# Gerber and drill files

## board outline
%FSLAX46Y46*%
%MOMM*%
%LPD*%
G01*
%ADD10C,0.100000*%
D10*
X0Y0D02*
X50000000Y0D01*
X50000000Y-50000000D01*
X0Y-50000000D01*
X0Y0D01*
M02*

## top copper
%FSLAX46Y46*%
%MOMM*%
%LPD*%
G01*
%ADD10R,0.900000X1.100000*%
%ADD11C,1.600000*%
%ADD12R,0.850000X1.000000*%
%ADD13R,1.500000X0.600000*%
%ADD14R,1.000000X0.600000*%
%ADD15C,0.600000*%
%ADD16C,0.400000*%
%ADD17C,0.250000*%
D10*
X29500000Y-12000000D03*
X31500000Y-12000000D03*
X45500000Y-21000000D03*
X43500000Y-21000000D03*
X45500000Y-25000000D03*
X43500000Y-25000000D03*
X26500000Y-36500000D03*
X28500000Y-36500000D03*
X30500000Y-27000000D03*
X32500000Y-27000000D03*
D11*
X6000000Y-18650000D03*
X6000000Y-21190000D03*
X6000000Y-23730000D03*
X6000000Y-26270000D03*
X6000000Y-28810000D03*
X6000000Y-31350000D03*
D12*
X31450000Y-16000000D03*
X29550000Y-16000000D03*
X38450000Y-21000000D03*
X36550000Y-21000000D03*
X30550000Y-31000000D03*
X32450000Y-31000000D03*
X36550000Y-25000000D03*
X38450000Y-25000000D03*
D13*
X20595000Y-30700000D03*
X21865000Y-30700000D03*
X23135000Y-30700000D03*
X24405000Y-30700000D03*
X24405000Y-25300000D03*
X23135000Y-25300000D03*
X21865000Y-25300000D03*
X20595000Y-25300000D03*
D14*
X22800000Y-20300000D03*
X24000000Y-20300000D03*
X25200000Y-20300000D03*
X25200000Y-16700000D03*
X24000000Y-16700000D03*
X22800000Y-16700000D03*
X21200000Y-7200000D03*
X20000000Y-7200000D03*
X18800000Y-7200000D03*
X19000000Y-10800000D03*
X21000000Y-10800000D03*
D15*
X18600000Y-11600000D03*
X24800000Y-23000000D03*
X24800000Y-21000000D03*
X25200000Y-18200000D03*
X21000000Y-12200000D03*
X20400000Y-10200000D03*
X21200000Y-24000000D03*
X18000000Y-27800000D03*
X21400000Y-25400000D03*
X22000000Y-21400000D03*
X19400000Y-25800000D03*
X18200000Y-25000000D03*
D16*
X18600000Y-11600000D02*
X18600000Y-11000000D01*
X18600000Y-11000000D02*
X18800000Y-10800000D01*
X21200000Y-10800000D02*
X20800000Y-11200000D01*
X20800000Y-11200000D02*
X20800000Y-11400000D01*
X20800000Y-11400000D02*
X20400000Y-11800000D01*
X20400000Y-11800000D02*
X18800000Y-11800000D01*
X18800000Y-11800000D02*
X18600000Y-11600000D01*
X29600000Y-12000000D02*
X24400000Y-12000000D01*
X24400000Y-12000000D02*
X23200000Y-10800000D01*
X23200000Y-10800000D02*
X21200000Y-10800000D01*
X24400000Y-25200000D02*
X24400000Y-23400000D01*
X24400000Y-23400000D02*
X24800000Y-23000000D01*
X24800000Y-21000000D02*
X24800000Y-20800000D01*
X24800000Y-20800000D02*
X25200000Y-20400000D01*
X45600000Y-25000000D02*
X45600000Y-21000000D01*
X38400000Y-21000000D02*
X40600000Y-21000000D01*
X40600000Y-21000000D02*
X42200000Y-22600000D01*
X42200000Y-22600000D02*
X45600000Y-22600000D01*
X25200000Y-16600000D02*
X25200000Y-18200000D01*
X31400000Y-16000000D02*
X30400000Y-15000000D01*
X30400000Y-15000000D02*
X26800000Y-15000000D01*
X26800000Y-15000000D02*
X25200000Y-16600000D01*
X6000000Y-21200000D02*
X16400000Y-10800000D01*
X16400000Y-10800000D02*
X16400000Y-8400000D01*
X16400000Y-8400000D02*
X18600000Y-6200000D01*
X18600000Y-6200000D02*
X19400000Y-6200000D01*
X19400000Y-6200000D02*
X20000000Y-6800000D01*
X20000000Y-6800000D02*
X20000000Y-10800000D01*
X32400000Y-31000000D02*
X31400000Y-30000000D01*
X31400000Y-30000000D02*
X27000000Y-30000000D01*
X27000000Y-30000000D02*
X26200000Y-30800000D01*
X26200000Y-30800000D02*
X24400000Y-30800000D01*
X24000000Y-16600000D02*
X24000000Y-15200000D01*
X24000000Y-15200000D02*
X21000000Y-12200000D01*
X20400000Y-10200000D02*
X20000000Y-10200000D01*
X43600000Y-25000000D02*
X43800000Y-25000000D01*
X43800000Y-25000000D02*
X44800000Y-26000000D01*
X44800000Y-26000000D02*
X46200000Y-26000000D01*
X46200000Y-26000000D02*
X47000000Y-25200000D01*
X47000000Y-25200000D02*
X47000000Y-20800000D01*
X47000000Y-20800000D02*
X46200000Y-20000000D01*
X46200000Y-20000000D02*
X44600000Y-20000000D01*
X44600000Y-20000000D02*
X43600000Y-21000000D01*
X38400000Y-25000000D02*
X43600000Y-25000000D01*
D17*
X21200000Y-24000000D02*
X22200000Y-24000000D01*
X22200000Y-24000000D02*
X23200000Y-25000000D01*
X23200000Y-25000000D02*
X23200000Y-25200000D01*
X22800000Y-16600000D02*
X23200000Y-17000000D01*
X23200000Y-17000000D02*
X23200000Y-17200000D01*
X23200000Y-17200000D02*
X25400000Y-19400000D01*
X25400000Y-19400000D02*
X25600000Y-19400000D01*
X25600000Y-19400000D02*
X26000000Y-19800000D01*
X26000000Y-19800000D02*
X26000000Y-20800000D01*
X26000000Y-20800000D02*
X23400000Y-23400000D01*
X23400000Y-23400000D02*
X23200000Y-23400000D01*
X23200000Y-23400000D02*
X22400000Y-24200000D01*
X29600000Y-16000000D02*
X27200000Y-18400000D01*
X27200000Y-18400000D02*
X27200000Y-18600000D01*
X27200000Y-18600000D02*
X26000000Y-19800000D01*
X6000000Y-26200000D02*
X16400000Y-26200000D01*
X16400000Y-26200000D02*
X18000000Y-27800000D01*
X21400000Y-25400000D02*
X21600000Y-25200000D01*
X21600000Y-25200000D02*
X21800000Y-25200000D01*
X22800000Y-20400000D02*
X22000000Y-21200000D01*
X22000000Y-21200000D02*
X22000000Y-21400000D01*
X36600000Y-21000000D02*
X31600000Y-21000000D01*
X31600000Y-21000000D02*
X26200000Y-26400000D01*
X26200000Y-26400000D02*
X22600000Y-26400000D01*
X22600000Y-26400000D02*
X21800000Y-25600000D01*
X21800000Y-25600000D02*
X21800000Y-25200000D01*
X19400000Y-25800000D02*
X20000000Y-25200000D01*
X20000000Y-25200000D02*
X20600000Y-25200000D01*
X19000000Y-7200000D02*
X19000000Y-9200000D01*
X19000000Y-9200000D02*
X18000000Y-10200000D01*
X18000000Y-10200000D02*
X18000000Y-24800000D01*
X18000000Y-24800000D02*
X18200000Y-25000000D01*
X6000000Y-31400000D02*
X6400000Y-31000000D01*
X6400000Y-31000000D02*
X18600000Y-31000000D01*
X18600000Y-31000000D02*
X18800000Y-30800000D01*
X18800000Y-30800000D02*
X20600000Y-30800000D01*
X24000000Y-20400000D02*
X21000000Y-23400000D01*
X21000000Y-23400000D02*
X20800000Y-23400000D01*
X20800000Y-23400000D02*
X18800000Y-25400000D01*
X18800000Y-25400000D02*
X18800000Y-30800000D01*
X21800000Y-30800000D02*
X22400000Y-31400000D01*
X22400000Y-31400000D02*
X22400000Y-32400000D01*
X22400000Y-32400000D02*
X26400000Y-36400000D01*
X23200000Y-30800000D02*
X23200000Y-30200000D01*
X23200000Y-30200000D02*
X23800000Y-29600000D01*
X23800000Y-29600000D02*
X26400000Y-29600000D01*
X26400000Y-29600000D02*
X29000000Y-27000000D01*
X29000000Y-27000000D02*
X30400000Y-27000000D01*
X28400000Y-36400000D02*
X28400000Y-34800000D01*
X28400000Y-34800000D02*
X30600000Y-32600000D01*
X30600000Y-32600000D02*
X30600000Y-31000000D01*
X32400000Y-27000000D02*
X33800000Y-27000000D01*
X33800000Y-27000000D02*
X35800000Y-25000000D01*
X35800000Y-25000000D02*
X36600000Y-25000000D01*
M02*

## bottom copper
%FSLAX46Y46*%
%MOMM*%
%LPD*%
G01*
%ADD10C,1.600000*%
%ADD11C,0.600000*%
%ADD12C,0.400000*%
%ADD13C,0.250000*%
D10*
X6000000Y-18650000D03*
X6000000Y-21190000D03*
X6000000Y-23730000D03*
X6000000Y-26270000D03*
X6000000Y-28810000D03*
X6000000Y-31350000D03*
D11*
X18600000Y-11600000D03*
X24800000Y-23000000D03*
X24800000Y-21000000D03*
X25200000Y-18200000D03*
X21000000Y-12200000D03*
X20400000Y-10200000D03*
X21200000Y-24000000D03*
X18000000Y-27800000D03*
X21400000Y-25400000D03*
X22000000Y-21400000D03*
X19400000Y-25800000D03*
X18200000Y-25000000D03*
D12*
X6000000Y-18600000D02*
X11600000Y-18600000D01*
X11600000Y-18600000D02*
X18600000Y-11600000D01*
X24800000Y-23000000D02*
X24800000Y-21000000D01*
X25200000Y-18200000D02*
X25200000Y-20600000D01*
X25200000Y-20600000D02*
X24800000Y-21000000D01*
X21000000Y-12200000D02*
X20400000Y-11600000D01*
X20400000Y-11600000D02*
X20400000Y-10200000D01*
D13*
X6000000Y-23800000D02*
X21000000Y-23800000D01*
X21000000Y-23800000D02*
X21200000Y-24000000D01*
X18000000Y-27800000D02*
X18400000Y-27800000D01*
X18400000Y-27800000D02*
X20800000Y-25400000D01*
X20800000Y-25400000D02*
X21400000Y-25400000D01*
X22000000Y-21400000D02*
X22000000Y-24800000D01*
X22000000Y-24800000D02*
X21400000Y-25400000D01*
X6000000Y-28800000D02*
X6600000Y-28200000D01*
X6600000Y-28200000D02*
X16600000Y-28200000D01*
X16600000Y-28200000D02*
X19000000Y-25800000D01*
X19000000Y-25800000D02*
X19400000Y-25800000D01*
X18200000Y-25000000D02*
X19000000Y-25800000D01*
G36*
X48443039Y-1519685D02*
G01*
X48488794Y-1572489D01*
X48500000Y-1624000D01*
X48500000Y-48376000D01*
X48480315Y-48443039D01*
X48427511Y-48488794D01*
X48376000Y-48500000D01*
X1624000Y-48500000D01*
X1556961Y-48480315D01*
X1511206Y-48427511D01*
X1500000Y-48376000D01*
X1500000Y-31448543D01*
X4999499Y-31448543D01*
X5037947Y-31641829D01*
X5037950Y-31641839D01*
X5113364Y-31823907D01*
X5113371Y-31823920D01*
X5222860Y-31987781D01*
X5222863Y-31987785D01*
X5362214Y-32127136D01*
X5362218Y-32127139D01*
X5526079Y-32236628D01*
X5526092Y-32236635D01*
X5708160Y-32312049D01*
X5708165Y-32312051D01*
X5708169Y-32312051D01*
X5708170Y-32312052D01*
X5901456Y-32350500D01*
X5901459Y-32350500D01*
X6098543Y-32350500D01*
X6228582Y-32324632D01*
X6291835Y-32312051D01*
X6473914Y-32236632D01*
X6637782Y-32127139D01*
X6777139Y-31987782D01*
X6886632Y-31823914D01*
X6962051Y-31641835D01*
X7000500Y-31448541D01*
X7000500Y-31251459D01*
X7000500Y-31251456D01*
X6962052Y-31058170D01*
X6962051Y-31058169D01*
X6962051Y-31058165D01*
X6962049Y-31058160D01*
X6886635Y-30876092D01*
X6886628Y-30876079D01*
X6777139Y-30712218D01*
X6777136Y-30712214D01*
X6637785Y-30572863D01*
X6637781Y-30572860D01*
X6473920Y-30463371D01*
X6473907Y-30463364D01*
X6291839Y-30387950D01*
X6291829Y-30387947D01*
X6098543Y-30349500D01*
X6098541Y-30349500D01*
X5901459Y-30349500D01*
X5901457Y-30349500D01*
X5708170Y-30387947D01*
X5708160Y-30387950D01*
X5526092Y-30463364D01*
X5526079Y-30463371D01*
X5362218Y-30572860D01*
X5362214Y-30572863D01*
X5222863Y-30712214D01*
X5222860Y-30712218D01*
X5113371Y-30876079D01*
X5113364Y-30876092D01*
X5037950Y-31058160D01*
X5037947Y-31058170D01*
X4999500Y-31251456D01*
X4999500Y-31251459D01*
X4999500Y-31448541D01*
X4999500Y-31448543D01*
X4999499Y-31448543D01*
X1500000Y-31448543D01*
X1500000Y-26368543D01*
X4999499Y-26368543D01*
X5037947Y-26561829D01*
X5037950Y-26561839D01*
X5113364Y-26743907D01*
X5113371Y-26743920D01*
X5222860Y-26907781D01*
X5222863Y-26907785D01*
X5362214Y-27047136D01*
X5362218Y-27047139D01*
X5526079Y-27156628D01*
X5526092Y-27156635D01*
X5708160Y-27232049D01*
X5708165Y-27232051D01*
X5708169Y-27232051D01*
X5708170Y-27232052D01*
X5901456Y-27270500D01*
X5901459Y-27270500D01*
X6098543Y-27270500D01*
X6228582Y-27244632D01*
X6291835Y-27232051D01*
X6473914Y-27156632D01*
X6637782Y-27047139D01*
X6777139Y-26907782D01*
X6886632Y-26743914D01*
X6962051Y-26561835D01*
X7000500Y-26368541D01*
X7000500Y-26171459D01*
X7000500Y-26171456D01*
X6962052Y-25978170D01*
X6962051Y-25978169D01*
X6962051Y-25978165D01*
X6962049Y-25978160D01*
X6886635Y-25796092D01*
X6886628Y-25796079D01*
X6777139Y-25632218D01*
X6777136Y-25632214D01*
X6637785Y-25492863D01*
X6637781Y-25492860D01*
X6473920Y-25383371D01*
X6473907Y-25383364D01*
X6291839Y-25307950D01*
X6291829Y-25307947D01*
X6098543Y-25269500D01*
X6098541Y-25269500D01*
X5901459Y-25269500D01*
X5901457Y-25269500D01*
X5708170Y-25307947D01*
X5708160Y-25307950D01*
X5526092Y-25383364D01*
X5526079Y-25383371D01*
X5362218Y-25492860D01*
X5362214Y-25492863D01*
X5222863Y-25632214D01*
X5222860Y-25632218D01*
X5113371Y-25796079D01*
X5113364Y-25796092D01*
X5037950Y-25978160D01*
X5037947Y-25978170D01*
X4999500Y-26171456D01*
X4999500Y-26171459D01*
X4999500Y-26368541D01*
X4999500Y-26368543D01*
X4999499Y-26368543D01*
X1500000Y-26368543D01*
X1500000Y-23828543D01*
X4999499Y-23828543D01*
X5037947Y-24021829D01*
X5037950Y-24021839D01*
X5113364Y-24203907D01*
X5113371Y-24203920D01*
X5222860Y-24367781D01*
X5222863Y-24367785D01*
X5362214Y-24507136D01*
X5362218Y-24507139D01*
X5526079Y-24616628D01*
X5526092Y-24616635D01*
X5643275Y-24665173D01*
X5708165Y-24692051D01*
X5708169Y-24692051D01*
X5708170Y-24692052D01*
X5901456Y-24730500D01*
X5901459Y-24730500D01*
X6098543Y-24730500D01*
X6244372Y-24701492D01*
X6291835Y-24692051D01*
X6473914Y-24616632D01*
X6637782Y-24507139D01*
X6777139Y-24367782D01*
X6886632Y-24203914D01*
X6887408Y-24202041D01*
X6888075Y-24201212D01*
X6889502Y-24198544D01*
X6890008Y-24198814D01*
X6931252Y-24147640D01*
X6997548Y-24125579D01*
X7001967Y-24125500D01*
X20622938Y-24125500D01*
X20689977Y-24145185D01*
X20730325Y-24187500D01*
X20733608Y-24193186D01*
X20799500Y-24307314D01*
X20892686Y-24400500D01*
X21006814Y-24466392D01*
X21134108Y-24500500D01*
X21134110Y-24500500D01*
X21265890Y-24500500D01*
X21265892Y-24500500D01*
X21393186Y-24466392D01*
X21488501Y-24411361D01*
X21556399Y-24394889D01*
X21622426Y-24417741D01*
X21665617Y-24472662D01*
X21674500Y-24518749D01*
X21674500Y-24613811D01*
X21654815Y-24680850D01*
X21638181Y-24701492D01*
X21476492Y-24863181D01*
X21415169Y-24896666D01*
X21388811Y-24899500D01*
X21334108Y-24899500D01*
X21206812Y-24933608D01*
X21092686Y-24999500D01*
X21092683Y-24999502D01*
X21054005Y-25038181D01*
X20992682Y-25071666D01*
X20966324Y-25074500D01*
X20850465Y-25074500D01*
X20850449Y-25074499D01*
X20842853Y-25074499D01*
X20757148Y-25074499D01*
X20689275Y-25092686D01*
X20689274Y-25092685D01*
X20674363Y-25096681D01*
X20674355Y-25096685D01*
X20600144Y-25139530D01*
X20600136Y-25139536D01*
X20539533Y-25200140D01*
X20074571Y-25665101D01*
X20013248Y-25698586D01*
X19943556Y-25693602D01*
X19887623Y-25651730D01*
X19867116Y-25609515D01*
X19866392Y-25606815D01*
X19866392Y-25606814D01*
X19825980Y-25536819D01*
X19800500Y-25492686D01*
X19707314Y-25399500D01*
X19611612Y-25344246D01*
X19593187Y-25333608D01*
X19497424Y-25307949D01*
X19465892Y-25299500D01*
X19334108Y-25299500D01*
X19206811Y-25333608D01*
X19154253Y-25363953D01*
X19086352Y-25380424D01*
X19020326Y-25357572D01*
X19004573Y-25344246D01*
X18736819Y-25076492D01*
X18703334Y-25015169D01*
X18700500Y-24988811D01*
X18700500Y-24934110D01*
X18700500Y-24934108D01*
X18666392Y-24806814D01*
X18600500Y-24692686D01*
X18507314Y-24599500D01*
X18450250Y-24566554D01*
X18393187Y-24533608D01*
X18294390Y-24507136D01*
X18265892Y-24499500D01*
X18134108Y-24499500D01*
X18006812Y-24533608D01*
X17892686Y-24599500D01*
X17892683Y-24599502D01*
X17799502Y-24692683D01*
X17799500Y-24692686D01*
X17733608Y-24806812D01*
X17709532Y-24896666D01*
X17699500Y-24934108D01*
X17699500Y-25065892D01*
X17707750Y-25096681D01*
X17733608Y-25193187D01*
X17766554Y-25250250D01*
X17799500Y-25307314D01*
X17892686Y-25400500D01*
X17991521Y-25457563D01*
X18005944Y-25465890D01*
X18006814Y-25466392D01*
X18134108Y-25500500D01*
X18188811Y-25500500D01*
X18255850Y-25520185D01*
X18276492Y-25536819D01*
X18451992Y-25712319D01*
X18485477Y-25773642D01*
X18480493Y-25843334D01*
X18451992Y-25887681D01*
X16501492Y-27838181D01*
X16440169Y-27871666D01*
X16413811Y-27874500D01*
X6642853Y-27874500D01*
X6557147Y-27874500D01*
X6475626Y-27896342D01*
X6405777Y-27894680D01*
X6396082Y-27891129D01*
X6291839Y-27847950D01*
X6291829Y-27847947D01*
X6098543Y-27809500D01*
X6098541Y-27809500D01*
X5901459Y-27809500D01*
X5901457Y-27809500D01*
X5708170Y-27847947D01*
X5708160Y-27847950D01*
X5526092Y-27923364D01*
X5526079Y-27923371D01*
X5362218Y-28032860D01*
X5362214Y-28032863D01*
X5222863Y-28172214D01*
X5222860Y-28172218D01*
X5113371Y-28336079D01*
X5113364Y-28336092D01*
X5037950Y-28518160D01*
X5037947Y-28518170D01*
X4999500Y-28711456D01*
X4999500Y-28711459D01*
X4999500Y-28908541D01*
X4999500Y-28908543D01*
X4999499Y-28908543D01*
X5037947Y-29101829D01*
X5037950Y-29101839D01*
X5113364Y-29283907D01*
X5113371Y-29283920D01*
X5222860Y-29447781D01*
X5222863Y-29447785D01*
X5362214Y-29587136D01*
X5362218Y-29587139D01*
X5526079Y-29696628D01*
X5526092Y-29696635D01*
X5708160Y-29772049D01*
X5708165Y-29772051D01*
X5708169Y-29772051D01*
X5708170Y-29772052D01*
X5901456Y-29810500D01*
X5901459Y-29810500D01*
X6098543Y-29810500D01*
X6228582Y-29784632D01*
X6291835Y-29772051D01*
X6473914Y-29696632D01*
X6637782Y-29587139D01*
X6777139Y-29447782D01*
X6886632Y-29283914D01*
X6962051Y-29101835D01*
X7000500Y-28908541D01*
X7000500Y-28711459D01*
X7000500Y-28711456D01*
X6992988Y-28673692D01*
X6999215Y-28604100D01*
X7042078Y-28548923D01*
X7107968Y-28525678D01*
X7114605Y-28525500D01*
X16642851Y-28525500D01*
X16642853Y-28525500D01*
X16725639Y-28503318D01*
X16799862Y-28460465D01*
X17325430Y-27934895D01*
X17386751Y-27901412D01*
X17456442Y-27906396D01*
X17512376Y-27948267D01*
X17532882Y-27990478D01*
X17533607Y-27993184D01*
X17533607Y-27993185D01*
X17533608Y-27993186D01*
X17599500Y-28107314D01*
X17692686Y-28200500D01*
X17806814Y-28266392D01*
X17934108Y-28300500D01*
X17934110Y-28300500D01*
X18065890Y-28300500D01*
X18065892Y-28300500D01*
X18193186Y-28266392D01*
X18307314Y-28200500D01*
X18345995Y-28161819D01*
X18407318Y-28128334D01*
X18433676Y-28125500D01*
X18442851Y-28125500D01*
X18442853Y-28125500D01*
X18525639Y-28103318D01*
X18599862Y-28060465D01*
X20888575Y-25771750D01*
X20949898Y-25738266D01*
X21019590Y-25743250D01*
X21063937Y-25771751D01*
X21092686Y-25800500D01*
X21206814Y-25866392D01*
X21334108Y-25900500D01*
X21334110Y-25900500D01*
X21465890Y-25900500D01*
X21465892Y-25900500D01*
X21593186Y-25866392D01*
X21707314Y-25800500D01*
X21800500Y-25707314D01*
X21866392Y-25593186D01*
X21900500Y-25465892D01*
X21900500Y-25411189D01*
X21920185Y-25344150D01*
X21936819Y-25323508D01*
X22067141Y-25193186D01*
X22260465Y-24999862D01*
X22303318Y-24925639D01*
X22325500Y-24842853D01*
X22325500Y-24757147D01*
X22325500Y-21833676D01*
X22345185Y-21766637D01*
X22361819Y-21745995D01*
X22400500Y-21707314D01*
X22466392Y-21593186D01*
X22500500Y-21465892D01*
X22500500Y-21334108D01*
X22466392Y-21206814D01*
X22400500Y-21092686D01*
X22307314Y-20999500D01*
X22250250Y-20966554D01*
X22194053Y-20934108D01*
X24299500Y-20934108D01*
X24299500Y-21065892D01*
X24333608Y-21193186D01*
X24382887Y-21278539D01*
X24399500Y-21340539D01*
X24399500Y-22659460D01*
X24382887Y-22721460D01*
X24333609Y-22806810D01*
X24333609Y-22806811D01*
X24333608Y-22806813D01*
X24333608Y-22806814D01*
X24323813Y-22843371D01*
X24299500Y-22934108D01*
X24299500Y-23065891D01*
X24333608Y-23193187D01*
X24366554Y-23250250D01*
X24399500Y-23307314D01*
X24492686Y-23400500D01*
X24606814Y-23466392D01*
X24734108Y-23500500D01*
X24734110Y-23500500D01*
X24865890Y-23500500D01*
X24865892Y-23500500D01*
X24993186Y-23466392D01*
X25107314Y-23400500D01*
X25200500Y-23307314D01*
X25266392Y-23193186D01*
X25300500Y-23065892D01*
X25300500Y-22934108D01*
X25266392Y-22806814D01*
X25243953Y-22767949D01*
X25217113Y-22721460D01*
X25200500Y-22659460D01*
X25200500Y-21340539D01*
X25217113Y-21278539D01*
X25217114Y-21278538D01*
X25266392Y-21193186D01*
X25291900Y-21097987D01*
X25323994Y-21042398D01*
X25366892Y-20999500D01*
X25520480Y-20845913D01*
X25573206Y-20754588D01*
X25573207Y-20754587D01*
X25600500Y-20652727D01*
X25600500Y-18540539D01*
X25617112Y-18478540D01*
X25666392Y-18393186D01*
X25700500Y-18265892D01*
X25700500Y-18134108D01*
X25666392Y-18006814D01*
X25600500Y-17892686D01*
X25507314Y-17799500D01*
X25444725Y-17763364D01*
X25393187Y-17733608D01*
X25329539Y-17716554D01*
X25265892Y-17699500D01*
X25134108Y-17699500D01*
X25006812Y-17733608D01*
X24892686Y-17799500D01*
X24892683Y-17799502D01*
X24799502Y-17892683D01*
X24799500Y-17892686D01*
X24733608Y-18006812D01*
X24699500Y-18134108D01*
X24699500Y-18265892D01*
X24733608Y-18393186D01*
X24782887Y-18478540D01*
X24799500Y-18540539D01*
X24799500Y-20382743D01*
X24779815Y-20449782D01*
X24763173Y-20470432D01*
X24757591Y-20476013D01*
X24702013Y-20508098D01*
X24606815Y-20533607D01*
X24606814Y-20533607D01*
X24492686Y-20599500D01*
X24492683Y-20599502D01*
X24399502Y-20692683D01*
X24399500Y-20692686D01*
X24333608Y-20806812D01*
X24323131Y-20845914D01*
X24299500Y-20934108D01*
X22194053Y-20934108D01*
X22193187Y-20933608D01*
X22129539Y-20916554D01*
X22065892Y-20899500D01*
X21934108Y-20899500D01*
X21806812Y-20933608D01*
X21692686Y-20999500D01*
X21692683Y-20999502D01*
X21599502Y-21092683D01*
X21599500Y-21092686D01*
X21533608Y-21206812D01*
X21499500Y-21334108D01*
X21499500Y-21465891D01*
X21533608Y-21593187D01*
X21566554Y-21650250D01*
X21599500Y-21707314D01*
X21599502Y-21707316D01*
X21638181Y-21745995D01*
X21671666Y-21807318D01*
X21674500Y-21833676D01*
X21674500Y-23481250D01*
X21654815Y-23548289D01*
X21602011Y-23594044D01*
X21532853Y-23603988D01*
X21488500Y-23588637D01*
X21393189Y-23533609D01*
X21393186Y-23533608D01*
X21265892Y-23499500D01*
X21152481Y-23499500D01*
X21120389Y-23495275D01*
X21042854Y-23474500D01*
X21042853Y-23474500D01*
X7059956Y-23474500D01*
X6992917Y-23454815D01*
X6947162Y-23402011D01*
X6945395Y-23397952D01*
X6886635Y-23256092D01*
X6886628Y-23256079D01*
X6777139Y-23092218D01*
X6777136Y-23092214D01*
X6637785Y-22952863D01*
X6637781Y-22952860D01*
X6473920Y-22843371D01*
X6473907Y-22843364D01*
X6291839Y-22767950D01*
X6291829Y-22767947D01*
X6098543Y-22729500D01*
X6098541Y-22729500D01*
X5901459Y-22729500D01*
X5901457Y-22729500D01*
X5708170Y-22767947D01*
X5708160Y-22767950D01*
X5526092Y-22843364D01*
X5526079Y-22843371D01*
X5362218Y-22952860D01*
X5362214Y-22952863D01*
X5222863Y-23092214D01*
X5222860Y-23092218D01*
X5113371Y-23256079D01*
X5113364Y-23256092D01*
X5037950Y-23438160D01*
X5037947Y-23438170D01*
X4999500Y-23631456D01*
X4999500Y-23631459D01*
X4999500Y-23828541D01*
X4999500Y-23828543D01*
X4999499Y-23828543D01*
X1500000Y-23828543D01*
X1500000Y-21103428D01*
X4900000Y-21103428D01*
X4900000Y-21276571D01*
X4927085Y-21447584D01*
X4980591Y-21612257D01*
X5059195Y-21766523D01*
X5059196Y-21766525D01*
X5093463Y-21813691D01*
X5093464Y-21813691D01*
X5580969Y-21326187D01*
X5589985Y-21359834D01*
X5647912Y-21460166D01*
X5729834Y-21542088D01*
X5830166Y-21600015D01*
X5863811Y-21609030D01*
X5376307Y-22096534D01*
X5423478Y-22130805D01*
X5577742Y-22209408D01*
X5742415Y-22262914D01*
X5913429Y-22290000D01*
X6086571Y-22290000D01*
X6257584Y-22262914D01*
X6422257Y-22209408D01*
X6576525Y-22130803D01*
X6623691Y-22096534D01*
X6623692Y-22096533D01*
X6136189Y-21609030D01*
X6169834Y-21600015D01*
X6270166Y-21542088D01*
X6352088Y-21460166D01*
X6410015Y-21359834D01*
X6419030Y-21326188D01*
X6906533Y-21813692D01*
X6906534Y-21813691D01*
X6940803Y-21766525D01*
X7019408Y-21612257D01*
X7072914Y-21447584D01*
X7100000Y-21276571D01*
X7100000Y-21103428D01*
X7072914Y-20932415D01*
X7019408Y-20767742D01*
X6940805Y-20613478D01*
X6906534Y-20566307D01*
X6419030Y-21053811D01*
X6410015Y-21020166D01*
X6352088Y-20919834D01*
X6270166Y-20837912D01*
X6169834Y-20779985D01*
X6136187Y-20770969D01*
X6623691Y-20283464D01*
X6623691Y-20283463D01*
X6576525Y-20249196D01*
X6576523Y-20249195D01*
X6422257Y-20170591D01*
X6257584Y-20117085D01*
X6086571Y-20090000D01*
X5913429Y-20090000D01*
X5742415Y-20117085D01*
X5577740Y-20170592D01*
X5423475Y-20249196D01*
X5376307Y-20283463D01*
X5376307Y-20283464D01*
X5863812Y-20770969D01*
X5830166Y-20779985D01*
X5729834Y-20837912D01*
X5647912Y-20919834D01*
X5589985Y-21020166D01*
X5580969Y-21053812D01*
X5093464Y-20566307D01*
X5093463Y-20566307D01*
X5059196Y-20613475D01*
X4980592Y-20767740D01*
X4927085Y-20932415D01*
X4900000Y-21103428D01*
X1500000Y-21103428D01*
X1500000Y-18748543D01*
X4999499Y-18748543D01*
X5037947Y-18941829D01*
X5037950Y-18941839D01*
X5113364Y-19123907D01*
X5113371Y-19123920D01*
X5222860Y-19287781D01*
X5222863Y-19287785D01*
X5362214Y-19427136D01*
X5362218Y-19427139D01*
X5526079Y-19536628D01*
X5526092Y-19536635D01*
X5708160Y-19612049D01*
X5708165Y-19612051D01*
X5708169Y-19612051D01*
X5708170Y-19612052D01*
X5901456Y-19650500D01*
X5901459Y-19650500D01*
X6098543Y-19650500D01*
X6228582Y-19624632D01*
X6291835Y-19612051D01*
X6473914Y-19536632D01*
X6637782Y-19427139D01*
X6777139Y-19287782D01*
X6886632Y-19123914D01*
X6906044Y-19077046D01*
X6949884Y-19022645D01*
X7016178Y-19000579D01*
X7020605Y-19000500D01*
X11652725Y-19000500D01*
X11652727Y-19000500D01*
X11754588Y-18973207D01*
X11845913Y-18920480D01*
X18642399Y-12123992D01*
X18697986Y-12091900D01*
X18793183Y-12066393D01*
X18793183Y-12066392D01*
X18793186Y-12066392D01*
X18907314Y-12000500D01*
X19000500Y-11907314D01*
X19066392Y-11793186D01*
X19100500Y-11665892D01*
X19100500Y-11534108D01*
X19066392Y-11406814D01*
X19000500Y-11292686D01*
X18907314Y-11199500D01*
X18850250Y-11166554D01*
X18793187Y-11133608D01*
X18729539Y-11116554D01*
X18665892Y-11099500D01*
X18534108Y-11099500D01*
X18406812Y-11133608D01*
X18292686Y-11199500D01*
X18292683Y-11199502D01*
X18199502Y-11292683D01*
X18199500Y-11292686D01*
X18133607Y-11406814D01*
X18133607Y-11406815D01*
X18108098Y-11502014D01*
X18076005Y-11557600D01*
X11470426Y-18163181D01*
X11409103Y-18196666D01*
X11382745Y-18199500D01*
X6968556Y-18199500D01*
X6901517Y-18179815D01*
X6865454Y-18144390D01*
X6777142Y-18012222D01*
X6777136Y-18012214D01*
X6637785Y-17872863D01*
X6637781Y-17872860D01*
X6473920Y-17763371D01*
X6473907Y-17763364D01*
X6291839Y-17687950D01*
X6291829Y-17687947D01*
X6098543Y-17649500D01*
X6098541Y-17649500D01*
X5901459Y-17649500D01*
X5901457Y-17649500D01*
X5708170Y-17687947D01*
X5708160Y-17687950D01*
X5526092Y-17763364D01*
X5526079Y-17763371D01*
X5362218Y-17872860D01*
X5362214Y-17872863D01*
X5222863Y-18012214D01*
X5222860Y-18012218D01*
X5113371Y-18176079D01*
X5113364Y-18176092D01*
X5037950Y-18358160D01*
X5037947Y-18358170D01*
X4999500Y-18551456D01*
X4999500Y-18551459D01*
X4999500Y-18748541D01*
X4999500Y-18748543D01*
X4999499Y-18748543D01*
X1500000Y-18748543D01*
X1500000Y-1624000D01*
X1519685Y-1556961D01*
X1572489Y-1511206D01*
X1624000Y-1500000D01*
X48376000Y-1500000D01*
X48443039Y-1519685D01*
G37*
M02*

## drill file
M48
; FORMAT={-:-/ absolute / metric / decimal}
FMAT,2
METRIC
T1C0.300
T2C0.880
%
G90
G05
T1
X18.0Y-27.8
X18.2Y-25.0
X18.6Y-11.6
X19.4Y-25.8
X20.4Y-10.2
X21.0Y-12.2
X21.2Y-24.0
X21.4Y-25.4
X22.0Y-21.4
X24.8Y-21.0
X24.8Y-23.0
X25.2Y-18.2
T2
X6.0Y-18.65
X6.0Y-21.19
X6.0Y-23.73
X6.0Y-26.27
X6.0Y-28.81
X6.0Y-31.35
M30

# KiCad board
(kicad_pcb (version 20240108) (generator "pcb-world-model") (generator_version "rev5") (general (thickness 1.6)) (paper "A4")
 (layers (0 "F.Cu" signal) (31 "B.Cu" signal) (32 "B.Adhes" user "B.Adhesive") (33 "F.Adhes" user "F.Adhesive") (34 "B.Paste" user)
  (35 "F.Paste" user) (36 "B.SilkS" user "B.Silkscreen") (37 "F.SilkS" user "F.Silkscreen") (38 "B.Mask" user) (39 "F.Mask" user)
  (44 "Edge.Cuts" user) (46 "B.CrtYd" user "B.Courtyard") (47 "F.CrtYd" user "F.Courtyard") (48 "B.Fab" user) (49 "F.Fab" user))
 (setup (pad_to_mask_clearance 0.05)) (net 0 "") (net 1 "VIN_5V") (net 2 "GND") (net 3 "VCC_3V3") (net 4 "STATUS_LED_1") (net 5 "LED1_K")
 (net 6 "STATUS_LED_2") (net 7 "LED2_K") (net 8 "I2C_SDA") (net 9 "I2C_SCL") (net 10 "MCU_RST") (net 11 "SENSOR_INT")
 (gr_rect (start 0.0 0.0) (end 50.0000 50.0000) (stroke (width 0.1) (type default)) (fill none) (layer "Edge.Cuts"))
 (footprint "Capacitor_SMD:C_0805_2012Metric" (layer "F.Cu") (at 30.5000 12.0000 0)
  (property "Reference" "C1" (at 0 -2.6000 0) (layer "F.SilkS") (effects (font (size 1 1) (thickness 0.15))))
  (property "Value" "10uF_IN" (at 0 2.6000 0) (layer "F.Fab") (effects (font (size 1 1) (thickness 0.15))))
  (pad "1" smd rect (at -1.0000 0.0000) (size 0.9000 1.1000) (layers "F.Cu" "F.Paste" "F.Mask") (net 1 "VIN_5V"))
  (pad "2" smd rect (at 1.0000 0.0000) (size 0.9000 1.1000) (layers "F.Cu" "F.Paste" "F.Mask") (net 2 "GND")))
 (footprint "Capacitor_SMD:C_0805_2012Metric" (layer "F.Cu") (at 44.5000 21.0000 180)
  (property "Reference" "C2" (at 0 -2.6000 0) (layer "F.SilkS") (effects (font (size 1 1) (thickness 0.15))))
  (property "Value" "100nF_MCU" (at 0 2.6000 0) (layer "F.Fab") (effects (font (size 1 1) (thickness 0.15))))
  (pad "1" smd rect (at -1.0000 0.0000) (size 0.9000 1.1000) (layers "F.Cu" "F.Paste" "F.Mask") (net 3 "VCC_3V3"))
  (pad "2" smd rect (at 1.0000 0.0000) (size 0.9000 1.1000) (layers "F.Cu" "F.Paste" "F.Mask") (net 2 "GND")))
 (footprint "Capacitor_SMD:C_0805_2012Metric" (layer "F.Cu") (at 44.5000 25.0000 180)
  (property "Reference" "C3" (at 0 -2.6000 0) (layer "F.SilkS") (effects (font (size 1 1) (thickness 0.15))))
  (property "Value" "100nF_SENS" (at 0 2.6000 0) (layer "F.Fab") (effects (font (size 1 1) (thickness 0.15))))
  (pad "1" smd rect (at -1.0000 0.0000) (size 0.9000 1.1000) (layers "F.Cu" "F.Paste" "F.Mask") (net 3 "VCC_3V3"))
  (pad "2" smd rect (at 1.0000 0.0000) (size 0.9000 1.1000) (layers "F.Cu" "F.Paste" "F.Mask") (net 2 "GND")))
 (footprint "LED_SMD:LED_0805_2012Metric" (layer "F.Cu") (at 27.5000 36.5000 0)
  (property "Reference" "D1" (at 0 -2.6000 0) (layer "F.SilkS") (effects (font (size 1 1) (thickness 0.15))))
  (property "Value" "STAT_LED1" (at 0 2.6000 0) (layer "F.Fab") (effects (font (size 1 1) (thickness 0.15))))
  (pad "1" smd rect (at -1.0000 0.0000) (size 0.9000 1.1000) (layers "F.Cu" "F.Paste" "F.Mask") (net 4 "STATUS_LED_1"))
  (pad "2" smd rect (at 1.0000 0.0000) (size 0.9000 1.1000) (layers "F.Cu" "F.Paste" "F.Mask") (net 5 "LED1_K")))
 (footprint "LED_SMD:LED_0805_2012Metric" (layer "F.Cu") (at 31.5000 27.0000 0)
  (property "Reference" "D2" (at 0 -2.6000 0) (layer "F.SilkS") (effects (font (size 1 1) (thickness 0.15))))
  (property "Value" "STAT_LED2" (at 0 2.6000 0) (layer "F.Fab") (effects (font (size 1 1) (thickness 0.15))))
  (pad "1" smd rect (at -1.0000 0.0000) (size 0.9000 1.1000) (layers "F.Cu" "F.Paste" "F.Mask") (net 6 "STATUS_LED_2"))
  (pad "2" smd rect (at 1.0000 0.0000) (size 0.9000 1.1000) (layers "F.Cu" "F.Paste" "F.Mask") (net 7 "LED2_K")))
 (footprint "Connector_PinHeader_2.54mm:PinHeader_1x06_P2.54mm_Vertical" (layer "F.Cu") (at 6.0000 25.0000 0) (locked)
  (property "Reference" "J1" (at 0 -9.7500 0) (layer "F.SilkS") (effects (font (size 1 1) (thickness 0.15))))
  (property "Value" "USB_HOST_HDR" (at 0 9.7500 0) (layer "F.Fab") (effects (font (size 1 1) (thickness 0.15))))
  (pad "1" thru_hole circle (at 0.0000 -6.3500) (size 1.6000 1.6000) (drill 0.8800) (layers "*.Cu" "*.Mask") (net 1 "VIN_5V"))
  (pad "2" thru_hole circle (at 0.0000 -3.8100) (size 1.6000 1.6000) (drill 0.8800) (layers "*.Cu" "*.Mask") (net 2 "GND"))
  (pad "3" thru_hole circle (at 0.0000 -1.2700) (size 1.6000 1.6000) (drill 0.8800) (layers "*.Cu" "*.Mask") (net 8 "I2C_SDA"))
  (pad "4" thru_hole circle (at 0.0000 1.2700) (size 1.6000 1.6000) (drill 0.8800) (layers "*.Cu" "*.Mask") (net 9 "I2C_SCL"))
  (pad "5" thru_hole circle (at 0.0000 3.8100) (size 1.6000 1.6000) (drill 0.8800) (layers "*.Cu" "*.Mask") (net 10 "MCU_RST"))
  (pad "6" thru_hole circle (at 0.0000 6.3500) (size 1.6000 1.6000) (drill 0.8800) (layers "*.Cu" "*.Mask") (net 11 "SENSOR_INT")))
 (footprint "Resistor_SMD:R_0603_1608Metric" (layer "F.Cu") (at 30.5000 16.0000 180)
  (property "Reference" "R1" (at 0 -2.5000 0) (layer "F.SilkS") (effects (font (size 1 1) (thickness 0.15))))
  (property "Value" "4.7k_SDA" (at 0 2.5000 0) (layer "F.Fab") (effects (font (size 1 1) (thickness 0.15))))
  (pad "1" smd rect (at -0.9500 0.0000) (size 0.8500 1.0000) (layers "F.Cu" "F.Paste" "F.Mask") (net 3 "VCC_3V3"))
  (pad "2" smd rect (at 0.9500 0.0000) (size 0.8500 1.0000) (layers "F.Cu" "F.Paste" "F.Mask") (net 8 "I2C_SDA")))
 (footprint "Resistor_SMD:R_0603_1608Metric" (layer "F.Cu") (at 37.5000 21.0000 180)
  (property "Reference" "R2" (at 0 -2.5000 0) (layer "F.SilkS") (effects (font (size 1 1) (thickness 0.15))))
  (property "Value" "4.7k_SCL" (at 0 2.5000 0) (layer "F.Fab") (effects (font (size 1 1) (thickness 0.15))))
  (pad "1" smd rect (at -0.9500 0.0000) (size 0.8500 1.0000) (layers "F.Cu" "F.Paste" "F.Mask") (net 3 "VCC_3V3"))
  (pad "2" smd rect (at 0.9500 0.0000) (size 0.8500 1.0000) (layers "F.Cu" "F.Paste" "F.Mask") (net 9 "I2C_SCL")))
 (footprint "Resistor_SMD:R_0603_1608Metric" (layer "F.Cu") (at 31.5000 31.0000 0)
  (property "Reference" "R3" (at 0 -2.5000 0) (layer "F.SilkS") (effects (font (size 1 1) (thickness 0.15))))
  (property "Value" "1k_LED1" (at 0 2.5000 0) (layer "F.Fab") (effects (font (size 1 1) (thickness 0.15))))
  (pad "1" smd rect (at -0.9500 0.0000) (size 0.8500 1.0000) (layers "F.Cu" "F.Paste" "F.Mask") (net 5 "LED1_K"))
  (pad "2" smd rect (at 0.9500 0.0000) (size 0.8500 1.0000) (layers "F.Cu" "F.Paste" "F.Mask") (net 2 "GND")))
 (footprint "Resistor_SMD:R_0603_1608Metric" (layer "F.Cu") (at 37.5000 25.0000 0)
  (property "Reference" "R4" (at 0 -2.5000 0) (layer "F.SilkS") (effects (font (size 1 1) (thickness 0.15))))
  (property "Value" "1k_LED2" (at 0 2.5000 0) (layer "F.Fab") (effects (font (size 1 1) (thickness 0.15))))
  (pad "1" smd rect (at -0.9500 0.0000) (size 0.8500 1.0000) (layers "F.Cu" "F.Paste" "F.Mask") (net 7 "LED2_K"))
  (pad "2" smd rect (at 0.9500 0.0000) (size 0.8500 1.0000) (layers "F.Cu" "F.Paste" "F.Mask") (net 2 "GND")))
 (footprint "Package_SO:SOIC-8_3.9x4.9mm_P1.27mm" (layer "F.Cu") (at 22.5000 28.0000 90)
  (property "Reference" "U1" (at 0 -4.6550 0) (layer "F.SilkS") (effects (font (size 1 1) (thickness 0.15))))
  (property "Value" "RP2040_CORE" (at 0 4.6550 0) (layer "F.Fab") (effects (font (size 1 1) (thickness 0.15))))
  (pad "1" smd rect (at -2.7000 -1.9050) (size 1.5000 0.6000) (layers "F.Cu" "F.Paste" "F.Mask") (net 3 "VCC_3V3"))
  (pad "2" smd rect (at -2.7000 -0.6350) (size 1.5000 0.6000) (layers "F.Cu" "F.Paste" "F.Mask") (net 8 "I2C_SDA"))
  (pad "3" smd rect (at -2.7000 0.6350) (size 1.5000 0.6000) (layers "F.Cu" "F.Paste" "F.Mask") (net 9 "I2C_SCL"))
  (pad "4" smd rect (at -2.7000 1.9050) (size 1.5000 0.6000) (layers "F.Cu" "F.Paste" "F.Mask") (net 10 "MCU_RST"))
  (pad "5" smd rect (at 2.7000 1.9050) (size 1.5000 0.6000) (layers "F.Cu" "F.Paste" "F.Mask") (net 11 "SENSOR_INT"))
  (pad "6" smd rect (at 2.7000 0.6350) (size 1.5000 0.6000) (layers "F.Cu" "F.Paste" "F.Mask") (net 4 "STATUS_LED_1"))
  (pad "7" smd rect (at 2.7000 -0.6350) (size 1.5000 0.6000) (layers "F.Cu" "F.Paste" "F.Mask") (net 6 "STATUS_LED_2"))
  (pad "8" smd rect (at 2.7000 -1.9050) (size 1.5000 0.6000) (layers "F.Cu" "F.Paste" "F.Mask") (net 2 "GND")))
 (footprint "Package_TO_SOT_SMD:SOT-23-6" (layer "F.Cu") (at 24.0000 18.5000 90)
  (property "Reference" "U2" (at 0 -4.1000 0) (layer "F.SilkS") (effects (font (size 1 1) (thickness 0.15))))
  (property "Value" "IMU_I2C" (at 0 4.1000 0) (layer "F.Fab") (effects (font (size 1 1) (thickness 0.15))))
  (pad "1" smd rect (at -1.8000 -1.2000) (size 1.0000 0.6000) (layers "F.Cu" "F.Paste" "F.Mask") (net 3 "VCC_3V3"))
  (pad "2" smd rect (at -1.8000 0.0000) (size 1.0000 0.6000) (layers "F.Cu" "F.Paste" "F.Mask") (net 2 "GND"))
  (pad "3" smd rect (at -1.8000 1.2000) (size 1.0000 0.6000) (layers "F.Cu" "F.Paste" "F.Mask") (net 8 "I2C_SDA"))
  (pad "4" smd rect (at 1.8000 1.2000) (size 1.0000 0.6000) (layers "F.Cu" "F.Paste" "F.Mask") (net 9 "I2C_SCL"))
  (pad "5" smd rect (at 1.8000 0.0000) (size 1.0000 0.6000) (layers "F.Cu" "F.Paste" "F.Mask") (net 11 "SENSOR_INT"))
  (pad "6" smd rect (at 1.8000 -1.2000) (size 1.0000 0.6000) (layers "F.Cu" "F.Paste" "F.Mask") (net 3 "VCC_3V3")))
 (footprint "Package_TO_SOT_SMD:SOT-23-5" (layer "F.Cu") (at 20.0000 9.0000 270)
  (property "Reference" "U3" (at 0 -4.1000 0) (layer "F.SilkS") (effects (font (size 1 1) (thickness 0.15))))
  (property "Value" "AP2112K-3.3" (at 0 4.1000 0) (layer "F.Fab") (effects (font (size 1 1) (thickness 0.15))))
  (pad "1" smd rect (at -1.8000 -1.2000) (size 1.0000 0.6000) (layers "F.Cu" "F.Paste" "F.Mask") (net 1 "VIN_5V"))
  (pad "2" smd rect (at -1.8000 0.0000) (size 1.0000 0.6000) (layers "F.Cu" "F.Paste" "F.Mask") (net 2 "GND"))
  (pad "3" smd rect (at -1.8000 1.2000) (size 1.0000 0.6000) (layers "F.Cu" "F.Paste" "F.Mask") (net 1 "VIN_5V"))
  (pad "4" smd rect (at 1.8000 1.0000) (size 1.0000 0.6000) (layers "F.Cu" "F.Paste" "F.Mask") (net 3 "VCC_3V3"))
  (pad "5" smd rect (at 1.8000 -1.0000) (size 1.0000 0.6000) (layers "F.Cu" "F.Paste" "F.Mask") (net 10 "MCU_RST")))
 (segment (start 6.0000 18.6000) (end 11.6000 18.6000) (width 0.4000) (layer "B.Cu") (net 1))
 (segment (start 11.6000 18.6000) (end 18.6000 11.6000) (width 0.4000) (layer "B.Cu") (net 1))
 (segment (start 18.6000 11.6000) (end 18.6000 11.0000) (width 0.4000) (layer "F.Cu") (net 1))
 (segment (start 18.6000 11.0000) (end 18.8000 10.8000) (width 0.4000) (layer "F.Cu") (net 1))
 (segment (start 21.2000 10.8000) (end 20.8000 11.2000) (width 0.4000) (layer "F.Cu") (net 1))
 (segment (start 20.8000 11.2000) (end 20.8000 11.4000) (width 0.4000) (layer "F.Cu") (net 1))
 (segment (start 20.8000 11.4000) (end 20.4000 11.8000) (width 0.4000) (layer "F.Cu") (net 1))
 (segment (start 20.4000 11.8000) (end 18.8000 11.8000) (width 0.4000) (layer "F.Cu") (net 1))
 (segment (start 18.8000 11.8000) (end 18.6000 11.6000) (width 0.4000) (layer "F.Cu") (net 1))
 (segment (start 29.6000 12.0000) (end 24.4000 12.0000) (width 0.4000) (layer "F.Cu") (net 1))
 (segment (start 24.4000 12.0000) (end 23.2000 10.8000) (width 0.4000) (layer "F.Cu") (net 1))
 (segment (start 23.2000 10.8000) (end 21.2000 10.8000) (width 0.4000) (layer "F.Cu") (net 1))
 (segment (start 24.4000 25.2000) (end 24.4000 23.4000) (width 0.4000) (layer "F.Cu") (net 3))
 (segment (start 24.4000 23.4000) (end 24.8000 23.0000) (width 0.4000) (layer "F.Cu") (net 3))
 (segment (start 24.8000 23.0000) (end 24.8000 21.0000) (width 0.4000) (layer "B.Cu") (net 3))
 (segment (start 24.8000 21.0000) (end 24.8000 20.8000) (width 0.4000) (layer "F.Cu") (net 3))
 (segment (start 24.8000 20.8000) (end 25.2000 20.4000) (width 0.4000) (layer "F.Cu") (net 3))
 (segment (start 45.6000 25.0000) (end 45.6000 21.0000) (width 0.4000) (layer "F.Cu") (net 3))
 (segment (start 38.4000 21.0000) (end 40.6000 21.0000) (width 0.4000) (layer "F.Cu") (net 3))
 (segment (start 40.6000 21.0000) (end 42.2000 22.6000) (width 0.4000) (layer "F.Cu") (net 3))
 (segment (start 42.2000 22.6000) (end 45.6000 22.6000) (width 0.4000) (layer "F.Cu") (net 3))
 (segment (start 25.2000 16.6000) (end 25.2000 18.2000) (width 0.4000) (layer "F.Cu") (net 3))
 (segment (start 25.2000 18.2000) (end 25.2000 20.6000) (width 0.4000) (layer "B.Cu") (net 3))
 (segment (start 25.2000 20.6000) (end 24.8000 21.0000) (width 0.4000) (layer "B.Cu") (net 3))
 (segment (start 31.4000 16.0000) (end 30.4000 15.0000) (width 0.4000) (layer "F.Cu") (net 3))
 (segment (start 30.4000 15.0000) (end 26.8000 15.0000) (width 0.4000) (layer "F.Cu") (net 3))
 (segment (start 26.8000 15.0000) (end 25.2000 16.6000) (width 0.4000) (layer "F.Cu") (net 3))
 (segment (start 6.0000 21.2000) (end 16.4000 10.8000) (width 0.4000) (layer "F.Cu") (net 2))
 (segment (start 16.4000 10.8000) (end 16.4000 8.4000) (width 0.4000) (layer "F.Cu") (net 2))
 (segment (start 16.4000 8.4000) (end 18.6000 6.2000) (width 0.4000) (layer "F.Cu") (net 2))
 (segment (start 18.6000 6.2000) (end 19.4000 6.2000) (width 0.4000) (layer "F.Cu") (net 2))
 (segment (start 19.4000 6.2000) (end 20.0000 6.8000) (width 0.4000) (layer "F.Cu") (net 2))
 (segment (start 20.0000 6.8000) (end 20.0000 10.8000) (width 0.4000) (layer "F.Cu") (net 2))
 (segment (start 32.4000 31.0000) (end 31.4000 30.0000) (width 0.4000) (layer "F.Cu") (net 2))
 (segment (start 31.4000 30.0000) (end 27.0000 30.0000) (width 0.4000) (layer "F.Cu") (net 2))
 (segment (start 27.0000 30.0000) (end 26.2000 30.8000) (width 0.4000) (layer "F.Cu") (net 2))
 (segment (start 26.2000 30.8000) (end 24.4000 30.8000) (width 0.4000) (layer "F.Cu") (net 2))
 (segment (start 24.0000 16.6000) (end 24.0000 15.2000) (width 0.4000) (layer "F.Cu") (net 2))
 (segment (start 24.0000 15.2000) (end 21.0000 12.2000) (width 0.4000) (layer "F.Cu") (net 2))
 (segment (start 21.0000 12.2000) (end 20.4000 11.6000) (width 0.4000) (layer "B.Cu") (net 2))
 (segment (start 20.4000 11.6000) (end 20.4000 10.2000) (width 0.4000) (layer "B.Cu") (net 2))
 (segment (start 20.4000 10.2000) (end 20.0000 10.2000) (width 0.4000) (layer "F.Cu") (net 2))
 (segment (start 43.6000 25.0000) (end 43.8000 25.0000) (width 0.4000) (layer "F.Cu") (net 2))
 (segment (start 43.8000 25.0000) (end 44.8000 26.0000) (width 0.4000) (layer "F.Cu") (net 2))
 (segment (start 44.8000 26.0000) (end 46.2000 26.0000) (width 0.4000) (layer "F.Cu") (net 2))
 (segment (start 46.2000 26.0000) (end 47.0000 25.2000) (width 0.4000) (layer "F.Cu") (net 2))
 (segment (start 47.0000 25.2000) (end 47.0000 20.8000) (width 0.4000) (layer "F.Cu") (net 2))
 (segment (start 47.0000 20.8000) (end 46.2000 20.0000) (width 0.4000) (layer "F.Cu") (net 2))
 (segment (start 46.2000 20.0000) (end 44.6000 20.0000) (width 0.4000) (layer "F.Cu") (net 2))
 (segment (start 44.6000 20.0000) (end 43.6000 21.0000) (width 0.4000) (layer "F.Cu") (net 2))
 (segment (start 38.4000 25.0000) (end 43.6000 25.0000) (width 0.4000) (layer "F.Cu") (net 2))
 (segment (start 6.0000 23.8000) (end 21.0000 23.8000) (width 0.2500) (layer "B.Cu") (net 8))
 (segment (start 21.0000 23.8000) (end 21.2000 24.0000) (width 0.2500) (layer "B.Cu") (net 8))
 (segment (start 21.2000 24.0000) (end 22.2000 24.0000) (width 0.2500) (layer "F.Cu") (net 8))
 (segment (start 22.2000 24.0000) (end 23.2000 25.0000) (width 0.2500) (layer "F.Cu") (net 8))
 (segment (start 23.2000 25.0000) (end 23.2000 25.2000) (width 0.2500) (layer "F.Cu") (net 8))
 (segment (start 22.8000 16.6000) (end 23.2000 17.0000) (width 0.2500) (layer "F.Cu") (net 8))
 (segment (start 23.2000 17.0000) (end 23.2000 17.2000) (width 0.2500) (layer "F.Cu") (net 8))
 (segment (start 23.2000 17.2000) (end 25.4000 19.4000) (width 0.2500) (layer "F.Cu") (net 8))
 (segment (start 25.4000 19.4000) (end 25.6000 19.4000) (width 0.2500) (layer "F.Cu") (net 8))
 (segment (start 25.6000 19.4000) (end 26.0000 19.8000) (width 0.2500) (layer "F.Cu") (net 8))
 (segment (start 26.0000 19.8000) (end 26.0000 20.8000) (width 0.2500) (layer "F.Cu") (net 8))
 (segment (start 26.0000 20.8000) (end 23.4000 23.4000) (width 0.2500) (layer "F.Cu") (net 8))
 (segment (start 23.4000 23.4000) (end 23.2000 23.4000) (width 0.2500) (layer "F.Cu") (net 8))
 (segment (start 23.2000 23.4000) (end 22.4000 24.2000) (width 0.2500) (layer "F.Cu") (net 8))
 (segment (start 29.6000 16.0000) (end 27.2000 18.4000) (width 0.2500) (layer "F.Cu") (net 8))
 (segment (start 27.2000 18.4000) (end 27.2000 18.6000) (width 0.2500) (layer "F.Cu") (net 8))
 (segment (start 27.2000 18.6000) (end 26.0000 19.8000) (width 0.2500) (layer "F.Cu") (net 8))
 (segment (start 6.0000 26.2000) (end 16.4000 26.2000) (width 0.2500) (layer "F.Cu") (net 9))
 (segment (start 16.4000 26.2000) (end 18.0000 27.8000) (width 0.2500) (layer "F.Cu") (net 9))
 (segment (start 18.0000 27.8000) (end 18.4000 27.8000) (width 0.2500) (layer "B.Cu") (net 9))
 (segment (start 18.4000 27.8000) (end 20.8000 25.4000) (width 0.2500) (layer "B.Cu") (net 9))
 (segment (start 20.8000 25.4000) (end 21.4000 25.4000) (width 0.2500) (layer "B.Cu") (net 9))
 (segment (start 21.4000 25.4000) (end 21.6000 25.2000) (width 0.2500) (layer "F.Cu") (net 9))
 (segment (start 21.6000 25.2000) (end 21.8000 25.2000) (width 0.2500) (layer "F.Cu") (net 9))
 (segment (start 22.8000 20.4000) (end 22.0000 21.2000) (width 0.2500) (layer "F.Cu") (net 9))
 (segment (start 22.0000 21.2000) (end 22.0000 21.4000) (width 0.2500) (layer "F.Cu") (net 9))
 (segment (start 22.0000 21.4000) (end 22.0000 24.8000) (width 0.2500) (layer "B.Cu") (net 9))
 (segment (start 22.0000 24.8000) (end 21.4000 25.4000) (width 0.2500) (layer "B.Cu") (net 9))
 (segment (start 36.6000 21.0000) (end 31.6000 21.0000) (width 0.2500) (layer "F.Cu") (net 9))
 (segment (start 31.6000 21.0000) (end 26.2000 26.4000) (width 0.2500) (layer "F.Cu") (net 9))
 (segment (start 26.2000 26.4000) (end 22.6000 26.4000) (width 0.2500) (layer "F.Cu") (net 9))
 (segment (start 22.6000 26.4000) (end 21.8000 25.6000) (width 0.2500) (layer "F.Cu") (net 9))
 (segment (start 21.8000 25.6000) (end 21.8000 25.2000) (width 0.2500) (layer "F.Cu") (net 9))
 (segment (start 6.0000 28.8000) (end 6.6000 28.2000) (width 0.2500) (layer "B.Cu") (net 10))
 (segment (start 6.6000 28.2000) (end 16.6000 28.2000) (width 0.2500) (layer "B.Cu") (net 10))
 (segment (start 16.6000 28.2000) (end 19.0000 25.8000) (width 0.2500) (layer "B.Cu") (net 10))
 (segment (start 19.0000 25.8000) (end 19.4000 25.8000) (width 0.2500) (layer "B.Cu") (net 10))
 (segment (start 19.4000 25.8000) (end 20.0000 25.2000) (width 0.2500) (layer "F.Cu") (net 10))
 (segment (start 20.0000 25.2000) (end 20.6000 25.2000) (width 0.2500) (layer "F.Cu") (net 10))
 (segment (start 19.0000 7.2000) (end 19.0000 9.2000) (width 0.2500) (layer "F.Cu") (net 10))
 (segment (start 19.0000 9.2000) (end 18.0000 10.2000) (width 0.2500) (layer "F.Cu") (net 10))
 (segment (start 18.0000 10.2000) (end 18.0000 24.8000) (width 0.2500) (layer "F.Cu") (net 10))
 (segment (start 18.0000 24.8000) (end 18.2000 25.0000) (width 0.2500) (layer "F.Cu") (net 10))
 (segment (start 18.2000 25.0000) (end 19.0000 25.8000) (width 0.2500) (layer "B.Cu") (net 10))
 (segment (start 6.0000 31.4000) (end 6.4000 31.0000) (width 0.2500) (layer "F.Cu") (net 11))
 (segment (start 6.4000 31.0000) (end 18.6000 31.0000) (width 0.2500) (layer "F.Cu") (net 11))
 (segment (start 18.6000 31.0000) (end 18.8000 30.8000) (width 0.2500) (layer "F.Cu") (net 11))
 (segment (start 18.8000 30.8000) (end 20.6000 30.8000) (width 0.2500) (layer "F.Cu") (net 11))
 (segment (start 24.0000 20.4000) (end 21.0000 23.4000) (width 0.2500) (layer "F.Cu") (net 11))
 (segment (start 21.0000 23.4000) (end 20.8000 23.4000) (width 0.2500) (layer "F.Cu") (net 11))
 (segment (start 20.8000 23.4000) (end 18.8000 25.4000) (width 0.2500) (layer "F.Cu") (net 11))
 (segment (start 18.8000 25.4000) (end 18.8000 30.8000) (width 0.2500) (layer "F.Cu") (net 11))
 (segment (start 21.8000 30.8000) (end 22.4000 31.4000) (width 0.2500) (layer "F.Cu") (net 4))
 (segment (start 22.4000 31.4000) (end 22.4000 32.4000) (width 0.2500) (layer "F.Cu") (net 4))
 (segment (start 22.4000 32.4000) (end 26.4000 36.4000) (width 0.2500) (layer "F.Cu") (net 4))
 (segment (start 23.2000 30.8000) (end 23.2000 30.2000) (width 0.2500) (layer "F.Cu") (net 6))
 (segment (start 23.2000 30.2000) (end 23.8000 29.6000) (width 0.2500) (layer "F.Cu") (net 6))
 (segment (start 23.8000 29.6000) (end 26.4000 29.6000) (width 0.2500) (layer "F.Cu") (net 6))
 (segment (start 26.4000 29.6000) (end 29.0000 27.0000) (width 0.2500) (layer "F.Cu") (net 6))
 (segment (start 29.0000 27.0000) (end 30.4000 27.0000) (width 0.2500) (layer "F.Cu") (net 6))
 (segment (start 28.4000 36.4000) (end 28.4000 34.8000) (width 0.2500) (layer "F.Cu") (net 5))
 (segment (start 28.4000 34.8000) (end 30.6000 32.6000) (width 0.2500) (layer "F.Cu") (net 5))
 (segment (start 30.6000 32.6000) (end 30.6000 31.0000) (width 0.2500) (layer "F.Cu") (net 5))
 (segment (start 32.4000 27.0000) (end 33.8000 27.0000) (width 0.2500) (layer "F.Cu") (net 7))
 (segment (start 33.8000 27.0000) (end 35.8000 25.0000) (width 0.2500) (layer "F.Cu") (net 7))
 (segment (start 35.8000 25.0000) (end 36.6000 25.0000) (width 0.2500) (layer "F.Cu") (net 7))
 (via (at 18.6000 11.6000) (size 0.6000) (drill 0.3000) (layers "F.Cu" "B.Cu") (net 1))
 (via (at 24.8000 23.0000) (size 0.6000) (drill 0.3000) (layers "F.Cu" "B.Cu") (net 3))
 (via (at 24.8000 21.0000) (size 0.6000) (drill 0.3000) (layers "F.Cu" "B.Cu") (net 3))
 (via (at 25.2000 18.2000) (size 0.6000) (drill 0.3000) (layers "F.Cu" "B.Cu") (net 3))
 (via (at 21.0000 12.2000) (size 0.6000) (drill 0.3000) (layers "F.Cu" "B.Cu") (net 2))
 (via (at 20.4000 10.2000) (size 0.6000) (drill 0.3000) (layers "F.Cu" "B.Cu") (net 2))
 (via (at 21.2000 24.0000) (size 0.6000) (drill 0.3000) (layers "F.Cu" "B.Cu") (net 8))
 (via (at 18.0000 27.8000) (size 0.6000) (drill 0.3000) (layers "F.Cu" "B.Cu") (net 9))
 (via (at 21.4000 25.4000) (size 0.6000) (drill 0.3000) (layers "F.Cu" "B.Cu") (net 9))
 (via (at 22.0000 21.4000) (size 0.6000) (drill 0.3000) (layers "F.Cu" "B.Cu") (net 9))
 (via (at 19.4000 25.8000) (size 0.6000) (drill 0.3000) (layers "F.Cu" "B.Cu") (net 10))
 (via (at 18.2000 25.0000) (size 0.6000) (drill 0.3000) (layers "F.Cu" "B.Cu") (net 10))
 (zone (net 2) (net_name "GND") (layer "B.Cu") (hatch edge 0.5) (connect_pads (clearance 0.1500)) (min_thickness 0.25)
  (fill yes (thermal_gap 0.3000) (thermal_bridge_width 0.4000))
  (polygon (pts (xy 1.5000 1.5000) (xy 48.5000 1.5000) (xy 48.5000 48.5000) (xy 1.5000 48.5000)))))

